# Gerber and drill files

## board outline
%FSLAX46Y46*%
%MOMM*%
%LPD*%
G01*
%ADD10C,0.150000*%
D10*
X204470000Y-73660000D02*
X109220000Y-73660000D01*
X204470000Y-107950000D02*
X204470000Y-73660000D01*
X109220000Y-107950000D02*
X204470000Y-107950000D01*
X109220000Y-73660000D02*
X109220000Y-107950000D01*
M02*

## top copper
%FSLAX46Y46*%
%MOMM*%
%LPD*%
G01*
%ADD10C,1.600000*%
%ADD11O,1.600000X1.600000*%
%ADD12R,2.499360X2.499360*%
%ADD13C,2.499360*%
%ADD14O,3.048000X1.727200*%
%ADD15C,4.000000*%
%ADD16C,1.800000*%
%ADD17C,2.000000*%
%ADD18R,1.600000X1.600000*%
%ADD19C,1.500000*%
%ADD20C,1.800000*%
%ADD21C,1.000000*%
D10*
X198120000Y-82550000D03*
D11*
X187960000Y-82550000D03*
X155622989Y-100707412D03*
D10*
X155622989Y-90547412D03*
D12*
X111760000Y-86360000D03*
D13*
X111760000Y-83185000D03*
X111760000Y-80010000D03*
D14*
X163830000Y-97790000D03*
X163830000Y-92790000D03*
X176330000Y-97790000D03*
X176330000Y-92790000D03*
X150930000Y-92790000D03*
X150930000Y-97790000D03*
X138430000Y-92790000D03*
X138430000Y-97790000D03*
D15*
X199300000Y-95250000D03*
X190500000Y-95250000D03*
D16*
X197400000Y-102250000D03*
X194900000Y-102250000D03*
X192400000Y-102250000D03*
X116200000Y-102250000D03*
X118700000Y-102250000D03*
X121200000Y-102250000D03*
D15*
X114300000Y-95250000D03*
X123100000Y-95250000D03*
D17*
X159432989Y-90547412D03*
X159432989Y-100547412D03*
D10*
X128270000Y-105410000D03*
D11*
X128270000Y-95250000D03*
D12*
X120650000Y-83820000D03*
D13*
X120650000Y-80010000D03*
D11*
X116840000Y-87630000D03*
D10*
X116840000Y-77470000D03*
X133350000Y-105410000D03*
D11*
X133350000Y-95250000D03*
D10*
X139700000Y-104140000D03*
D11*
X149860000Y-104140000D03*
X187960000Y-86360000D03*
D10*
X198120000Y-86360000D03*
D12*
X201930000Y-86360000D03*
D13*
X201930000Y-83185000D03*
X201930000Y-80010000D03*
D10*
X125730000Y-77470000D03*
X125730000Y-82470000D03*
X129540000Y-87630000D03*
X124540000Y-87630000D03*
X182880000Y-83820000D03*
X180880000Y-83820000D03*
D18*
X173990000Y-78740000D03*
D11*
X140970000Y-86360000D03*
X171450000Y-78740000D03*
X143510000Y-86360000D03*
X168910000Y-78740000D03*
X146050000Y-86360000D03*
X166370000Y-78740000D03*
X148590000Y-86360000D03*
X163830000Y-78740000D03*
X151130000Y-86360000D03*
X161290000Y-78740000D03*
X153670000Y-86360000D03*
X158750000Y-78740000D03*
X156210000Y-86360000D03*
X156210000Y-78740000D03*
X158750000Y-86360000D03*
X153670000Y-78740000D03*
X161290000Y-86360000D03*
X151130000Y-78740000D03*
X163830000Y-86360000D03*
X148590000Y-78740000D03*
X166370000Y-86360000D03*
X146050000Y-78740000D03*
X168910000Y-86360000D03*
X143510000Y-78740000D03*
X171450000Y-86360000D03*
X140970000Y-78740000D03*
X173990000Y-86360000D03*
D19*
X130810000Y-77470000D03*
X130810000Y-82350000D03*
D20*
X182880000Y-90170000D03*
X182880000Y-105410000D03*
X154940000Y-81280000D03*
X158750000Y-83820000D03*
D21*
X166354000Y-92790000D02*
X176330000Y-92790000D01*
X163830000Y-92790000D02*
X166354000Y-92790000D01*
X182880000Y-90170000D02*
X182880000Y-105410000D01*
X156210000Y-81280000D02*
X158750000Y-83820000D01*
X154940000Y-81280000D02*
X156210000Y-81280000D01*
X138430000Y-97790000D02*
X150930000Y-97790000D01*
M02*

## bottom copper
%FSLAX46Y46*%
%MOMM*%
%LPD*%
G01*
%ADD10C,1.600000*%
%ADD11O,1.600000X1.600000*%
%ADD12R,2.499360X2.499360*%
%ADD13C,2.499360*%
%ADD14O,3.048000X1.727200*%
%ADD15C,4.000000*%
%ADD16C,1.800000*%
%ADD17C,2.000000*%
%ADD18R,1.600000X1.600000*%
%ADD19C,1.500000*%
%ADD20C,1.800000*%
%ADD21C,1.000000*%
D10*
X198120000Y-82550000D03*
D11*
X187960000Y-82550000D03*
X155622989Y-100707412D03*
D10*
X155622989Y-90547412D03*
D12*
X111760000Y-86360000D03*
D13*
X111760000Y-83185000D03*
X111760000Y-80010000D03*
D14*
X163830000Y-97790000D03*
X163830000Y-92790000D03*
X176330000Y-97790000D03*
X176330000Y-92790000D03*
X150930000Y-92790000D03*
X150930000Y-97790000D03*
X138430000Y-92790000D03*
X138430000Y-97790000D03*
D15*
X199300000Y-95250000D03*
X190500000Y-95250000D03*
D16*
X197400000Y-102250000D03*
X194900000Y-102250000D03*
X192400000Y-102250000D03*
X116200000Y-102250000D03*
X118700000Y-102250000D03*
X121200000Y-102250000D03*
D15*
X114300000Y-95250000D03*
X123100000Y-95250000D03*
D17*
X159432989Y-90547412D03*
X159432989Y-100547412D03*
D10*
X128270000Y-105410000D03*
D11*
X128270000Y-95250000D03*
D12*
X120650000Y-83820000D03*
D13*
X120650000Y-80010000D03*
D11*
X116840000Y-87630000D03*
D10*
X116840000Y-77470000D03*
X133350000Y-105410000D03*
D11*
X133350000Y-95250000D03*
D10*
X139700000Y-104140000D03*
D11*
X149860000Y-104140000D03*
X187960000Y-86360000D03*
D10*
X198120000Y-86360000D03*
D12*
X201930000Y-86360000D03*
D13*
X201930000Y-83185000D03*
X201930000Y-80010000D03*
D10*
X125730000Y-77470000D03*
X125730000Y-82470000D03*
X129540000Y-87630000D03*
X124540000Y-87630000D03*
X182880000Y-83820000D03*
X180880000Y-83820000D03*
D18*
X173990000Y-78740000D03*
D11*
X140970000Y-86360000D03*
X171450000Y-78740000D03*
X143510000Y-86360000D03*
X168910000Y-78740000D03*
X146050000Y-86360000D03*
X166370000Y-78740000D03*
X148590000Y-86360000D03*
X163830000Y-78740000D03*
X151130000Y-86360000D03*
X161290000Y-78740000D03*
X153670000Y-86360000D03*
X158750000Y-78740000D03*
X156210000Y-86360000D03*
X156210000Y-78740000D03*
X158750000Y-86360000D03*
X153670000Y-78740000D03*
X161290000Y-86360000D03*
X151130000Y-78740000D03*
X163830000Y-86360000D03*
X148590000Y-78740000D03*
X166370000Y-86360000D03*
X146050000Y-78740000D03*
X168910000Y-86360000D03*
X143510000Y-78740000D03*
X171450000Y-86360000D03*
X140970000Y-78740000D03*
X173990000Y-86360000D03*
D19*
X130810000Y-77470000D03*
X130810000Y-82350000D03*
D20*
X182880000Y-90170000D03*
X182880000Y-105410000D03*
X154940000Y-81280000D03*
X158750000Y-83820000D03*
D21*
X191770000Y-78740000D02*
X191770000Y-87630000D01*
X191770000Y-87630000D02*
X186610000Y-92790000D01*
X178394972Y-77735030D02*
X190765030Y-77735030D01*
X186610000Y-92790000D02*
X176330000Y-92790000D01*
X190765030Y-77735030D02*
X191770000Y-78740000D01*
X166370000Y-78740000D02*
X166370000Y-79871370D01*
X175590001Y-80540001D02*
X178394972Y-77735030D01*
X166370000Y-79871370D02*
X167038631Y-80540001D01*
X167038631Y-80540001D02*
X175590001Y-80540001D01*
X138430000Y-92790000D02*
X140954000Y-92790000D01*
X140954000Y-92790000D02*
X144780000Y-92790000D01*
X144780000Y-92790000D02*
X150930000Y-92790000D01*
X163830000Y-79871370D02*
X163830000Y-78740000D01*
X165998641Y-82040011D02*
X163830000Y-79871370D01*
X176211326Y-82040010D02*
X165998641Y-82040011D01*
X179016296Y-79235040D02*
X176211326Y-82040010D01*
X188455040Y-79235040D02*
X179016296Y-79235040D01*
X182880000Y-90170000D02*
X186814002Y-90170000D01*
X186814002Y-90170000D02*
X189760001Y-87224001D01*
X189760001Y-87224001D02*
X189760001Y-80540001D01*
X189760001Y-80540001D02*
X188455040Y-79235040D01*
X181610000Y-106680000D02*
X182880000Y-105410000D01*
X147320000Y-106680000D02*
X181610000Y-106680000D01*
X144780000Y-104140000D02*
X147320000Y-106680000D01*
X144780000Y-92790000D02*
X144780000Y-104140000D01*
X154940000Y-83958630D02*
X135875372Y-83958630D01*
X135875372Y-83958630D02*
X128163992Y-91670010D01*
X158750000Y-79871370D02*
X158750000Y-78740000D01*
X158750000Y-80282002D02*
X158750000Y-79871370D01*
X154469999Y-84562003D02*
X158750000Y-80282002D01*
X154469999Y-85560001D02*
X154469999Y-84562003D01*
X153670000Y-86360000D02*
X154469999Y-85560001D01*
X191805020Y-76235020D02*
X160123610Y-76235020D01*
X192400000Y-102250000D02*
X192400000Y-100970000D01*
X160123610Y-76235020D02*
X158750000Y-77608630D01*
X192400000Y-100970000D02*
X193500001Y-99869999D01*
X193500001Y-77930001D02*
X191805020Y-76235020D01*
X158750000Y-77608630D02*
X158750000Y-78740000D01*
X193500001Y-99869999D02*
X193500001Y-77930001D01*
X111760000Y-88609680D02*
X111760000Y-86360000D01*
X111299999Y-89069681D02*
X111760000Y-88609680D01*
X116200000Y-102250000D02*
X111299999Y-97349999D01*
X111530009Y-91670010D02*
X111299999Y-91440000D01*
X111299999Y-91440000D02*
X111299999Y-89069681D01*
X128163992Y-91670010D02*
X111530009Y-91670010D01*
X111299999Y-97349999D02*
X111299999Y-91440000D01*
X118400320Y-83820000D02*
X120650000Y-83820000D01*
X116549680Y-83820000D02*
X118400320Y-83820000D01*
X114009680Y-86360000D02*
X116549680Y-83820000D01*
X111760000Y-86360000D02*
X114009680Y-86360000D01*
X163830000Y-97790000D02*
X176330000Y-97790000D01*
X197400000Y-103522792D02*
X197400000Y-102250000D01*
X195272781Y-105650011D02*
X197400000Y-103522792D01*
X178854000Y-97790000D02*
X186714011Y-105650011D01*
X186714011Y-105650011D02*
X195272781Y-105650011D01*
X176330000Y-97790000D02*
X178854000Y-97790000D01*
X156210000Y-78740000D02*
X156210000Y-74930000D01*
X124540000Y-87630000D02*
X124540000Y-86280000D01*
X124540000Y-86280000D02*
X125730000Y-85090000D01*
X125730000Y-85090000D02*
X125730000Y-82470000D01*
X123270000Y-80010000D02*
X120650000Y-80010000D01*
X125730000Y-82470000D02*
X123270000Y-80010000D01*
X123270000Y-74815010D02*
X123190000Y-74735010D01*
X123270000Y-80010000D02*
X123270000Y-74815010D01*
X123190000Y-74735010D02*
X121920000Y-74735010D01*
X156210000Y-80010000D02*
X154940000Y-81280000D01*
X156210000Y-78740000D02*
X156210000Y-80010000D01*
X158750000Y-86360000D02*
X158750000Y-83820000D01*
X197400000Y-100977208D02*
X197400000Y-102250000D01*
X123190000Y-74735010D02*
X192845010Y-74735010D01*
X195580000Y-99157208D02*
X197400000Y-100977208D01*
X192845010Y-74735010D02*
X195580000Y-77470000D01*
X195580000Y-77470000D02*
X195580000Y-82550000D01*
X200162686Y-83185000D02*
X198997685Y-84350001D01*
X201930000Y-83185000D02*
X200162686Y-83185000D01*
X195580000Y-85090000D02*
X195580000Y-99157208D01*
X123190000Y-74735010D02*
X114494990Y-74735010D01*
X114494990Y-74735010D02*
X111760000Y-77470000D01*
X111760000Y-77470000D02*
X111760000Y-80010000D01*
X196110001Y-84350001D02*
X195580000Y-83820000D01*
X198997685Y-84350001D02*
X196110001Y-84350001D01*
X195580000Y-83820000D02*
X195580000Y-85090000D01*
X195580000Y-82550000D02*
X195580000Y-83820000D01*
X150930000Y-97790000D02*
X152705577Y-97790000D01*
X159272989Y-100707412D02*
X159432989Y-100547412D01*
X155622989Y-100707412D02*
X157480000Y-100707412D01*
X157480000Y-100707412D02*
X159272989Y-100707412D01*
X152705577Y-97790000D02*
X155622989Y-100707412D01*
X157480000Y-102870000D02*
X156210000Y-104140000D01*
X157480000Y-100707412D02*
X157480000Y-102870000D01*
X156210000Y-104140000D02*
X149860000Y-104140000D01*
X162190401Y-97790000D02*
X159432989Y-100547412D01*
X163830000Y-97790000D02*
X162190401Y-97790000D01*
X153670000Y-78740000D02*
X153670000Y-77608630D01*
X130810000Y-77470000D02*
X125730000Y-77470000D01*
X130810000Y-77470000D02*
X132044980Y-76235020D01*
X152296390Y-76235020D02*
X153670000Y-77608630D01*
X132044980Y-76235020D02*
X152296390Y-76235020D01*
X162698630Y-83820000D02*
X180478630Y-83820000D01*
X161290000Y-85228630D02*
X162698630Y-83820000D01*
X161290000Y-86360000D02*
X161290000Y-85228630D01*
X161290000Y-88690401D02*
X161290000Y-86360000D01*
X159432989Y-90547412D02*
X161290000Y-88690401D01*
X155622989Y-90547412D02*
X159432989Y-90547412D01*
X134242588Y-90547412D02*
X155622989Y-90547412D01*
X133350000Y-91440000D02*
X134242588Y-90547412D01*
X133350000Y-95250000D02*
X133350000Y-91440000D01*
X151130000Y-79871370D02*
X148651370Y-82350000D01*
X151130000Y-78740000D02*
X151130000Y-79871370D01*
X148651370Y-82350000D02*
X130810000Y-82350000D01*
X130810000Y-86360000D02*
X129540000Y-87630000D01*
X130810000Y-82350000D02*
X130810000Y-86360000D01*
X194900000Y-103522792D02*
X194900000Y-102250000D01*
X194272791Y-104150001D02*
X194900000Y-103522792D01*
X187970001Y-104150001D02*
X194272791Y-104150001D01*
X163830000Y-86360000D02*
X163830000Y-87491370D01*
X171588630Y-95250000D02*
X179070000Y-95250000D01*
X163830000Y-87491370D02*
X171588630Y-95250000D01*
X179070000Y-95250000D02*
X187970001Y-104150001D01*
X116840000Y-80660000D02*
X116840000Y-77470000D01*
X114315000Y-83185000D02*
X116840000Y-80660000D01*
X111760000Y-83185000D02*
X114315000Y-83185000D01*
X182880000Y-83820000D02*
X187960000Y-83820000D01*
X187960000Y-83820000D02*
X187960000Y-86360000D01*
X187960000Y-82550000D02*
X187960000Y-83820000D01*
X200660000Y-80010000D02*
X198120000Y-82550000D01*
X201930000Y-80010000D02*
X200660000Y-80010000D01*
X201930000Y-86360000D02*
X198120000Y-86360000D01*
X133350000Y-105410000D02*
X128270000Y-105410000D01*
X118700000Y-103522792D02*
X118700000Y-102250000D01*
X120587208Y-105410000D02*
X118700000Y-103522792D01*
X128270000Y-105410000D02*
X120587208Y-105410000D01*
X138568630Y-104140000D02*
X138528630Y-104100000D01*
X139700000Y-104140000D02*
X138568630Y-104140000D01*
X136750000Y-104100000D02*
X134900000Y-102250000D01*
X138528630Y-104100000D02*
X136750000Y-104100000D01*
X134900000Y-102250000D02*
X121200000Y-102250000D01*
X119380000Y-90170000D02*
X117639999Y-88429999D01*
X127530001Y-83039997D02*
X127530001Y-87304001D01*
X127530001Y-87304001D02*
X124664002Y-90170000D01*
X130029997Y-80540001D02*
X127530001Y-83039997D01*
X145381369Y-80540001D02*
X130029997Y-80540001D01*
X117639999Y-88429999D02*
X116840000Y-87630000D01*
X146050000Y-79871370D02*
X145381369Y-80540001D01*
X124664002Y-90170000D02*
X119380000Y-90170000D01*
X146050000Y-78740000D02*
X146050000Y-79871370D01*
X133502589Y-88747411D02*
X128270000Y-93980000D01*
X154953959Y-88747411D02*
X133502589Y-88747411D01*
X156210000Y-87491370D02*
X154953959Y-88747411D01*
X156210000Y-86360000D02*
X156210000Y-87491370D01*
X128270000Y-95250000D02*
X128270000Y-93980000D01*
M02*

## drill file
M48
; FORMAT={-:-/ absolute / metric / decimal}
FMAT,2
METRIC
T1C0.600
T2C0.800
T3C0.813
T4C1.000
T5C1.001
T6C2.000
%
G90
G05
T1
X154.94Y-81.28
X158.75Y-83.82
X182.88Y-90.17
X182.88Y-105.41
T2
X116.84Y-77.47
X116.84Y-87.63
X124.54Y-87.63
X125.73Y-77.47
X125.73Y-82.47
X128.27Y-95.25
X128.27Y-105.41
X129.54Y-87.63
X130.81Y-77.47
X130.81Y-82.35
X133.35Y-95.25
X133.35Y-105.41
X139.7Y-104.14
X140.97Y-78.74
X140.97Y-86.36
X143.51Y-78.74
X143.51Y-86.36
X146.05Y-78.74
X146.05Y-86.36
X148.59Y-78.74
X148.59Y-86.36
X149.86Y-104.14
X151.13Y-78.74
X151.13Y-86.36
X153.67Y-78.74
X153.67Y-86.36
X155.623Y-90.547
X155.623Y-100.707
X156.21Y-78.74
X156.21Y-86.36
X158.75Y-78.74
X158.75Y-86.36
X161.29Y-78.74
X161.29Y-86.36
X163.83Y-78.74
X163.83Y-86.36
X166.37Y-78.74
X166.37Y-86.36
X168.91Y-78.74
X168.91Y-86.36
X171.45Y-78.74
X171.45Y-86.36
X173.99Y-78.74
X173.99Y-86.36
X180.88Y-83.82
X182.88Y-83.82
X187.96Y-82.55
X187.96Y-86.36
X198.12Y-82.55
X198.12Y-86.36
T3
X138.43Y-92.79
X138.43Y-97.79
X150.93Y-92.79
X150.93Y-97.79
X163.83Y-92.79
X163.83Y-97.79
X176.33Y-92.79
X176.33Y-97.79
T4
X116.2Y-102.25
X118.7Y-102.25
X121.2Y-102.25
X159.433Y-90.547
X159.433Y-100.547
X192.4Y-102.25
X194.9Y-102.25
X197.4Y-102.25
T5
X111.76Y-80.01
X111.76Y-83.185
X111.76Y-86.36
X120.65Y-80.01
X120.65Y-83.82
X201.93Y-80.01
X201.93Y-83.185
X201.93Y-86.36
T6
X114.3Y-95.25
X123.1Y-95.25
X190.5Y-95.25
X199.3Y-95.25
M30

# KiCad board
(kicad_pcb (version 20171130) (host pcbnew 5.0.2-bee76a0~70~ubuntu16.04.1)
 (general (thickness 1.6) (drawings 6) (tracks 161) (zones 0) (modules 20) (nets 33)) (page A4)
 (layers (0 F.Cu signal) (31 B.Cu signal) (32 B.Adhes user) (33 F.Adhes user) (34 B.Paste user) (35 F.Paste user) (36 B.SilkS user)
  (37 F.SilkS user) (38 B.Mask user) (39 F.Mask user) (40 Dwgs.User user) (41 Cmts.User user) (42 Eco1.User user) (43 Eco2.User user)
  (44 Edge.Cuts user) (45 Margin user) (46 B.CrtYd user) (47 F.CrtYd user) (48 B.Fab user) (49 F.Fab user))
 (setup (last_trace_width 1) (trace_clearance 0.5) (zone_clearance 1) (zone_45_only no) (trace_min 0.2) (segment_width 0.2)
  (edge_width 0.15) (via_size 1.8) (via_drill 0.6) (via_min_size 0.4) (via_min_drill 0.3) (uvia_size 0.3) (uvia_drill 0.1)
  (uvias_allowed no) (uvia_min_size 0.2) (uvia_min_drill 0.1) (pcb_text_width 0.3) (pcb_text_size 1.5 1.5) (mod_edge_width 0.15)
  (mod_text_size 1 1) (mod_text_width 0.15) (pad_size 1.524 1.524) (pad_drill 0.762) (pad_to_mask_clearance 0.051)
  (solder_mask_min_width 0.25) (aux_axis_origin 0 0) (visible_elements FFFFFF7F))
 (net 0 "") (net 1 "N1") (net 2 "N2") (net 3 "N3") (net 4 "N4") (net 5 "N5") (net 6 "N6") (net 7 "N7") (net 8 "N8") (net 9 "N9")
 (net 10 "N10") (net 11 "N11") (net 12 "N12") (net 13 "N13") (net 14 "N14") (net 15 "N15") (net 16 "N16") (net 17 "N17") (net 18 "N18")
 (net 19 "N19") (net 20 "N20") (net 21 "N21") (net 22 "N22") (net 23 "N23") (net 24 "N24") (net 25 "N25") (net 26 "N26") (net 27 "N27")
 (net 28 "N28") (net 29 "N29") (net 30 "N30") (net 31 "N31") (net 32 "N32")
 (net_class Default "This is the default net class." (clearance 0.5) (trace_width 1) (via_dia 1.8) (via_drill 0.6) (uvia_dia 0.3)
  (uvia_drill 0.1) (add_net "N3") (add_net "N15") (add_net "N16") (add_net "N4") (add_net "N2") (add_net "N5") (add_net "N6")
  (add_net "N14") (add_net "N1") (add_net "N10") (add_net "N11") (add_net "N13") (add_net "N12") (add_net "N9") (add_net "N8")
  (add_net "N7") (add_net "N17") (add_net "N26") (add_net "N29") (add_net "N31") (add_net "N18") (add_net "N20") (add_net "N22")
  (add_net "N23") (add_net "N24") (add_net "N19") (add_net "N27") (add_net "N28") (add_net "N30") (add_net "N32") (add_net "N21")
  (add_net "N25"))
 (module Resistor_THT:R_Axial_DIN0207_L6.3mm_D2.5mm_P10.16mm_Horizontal (layer F.Cu) (at 198.12 82.55 180)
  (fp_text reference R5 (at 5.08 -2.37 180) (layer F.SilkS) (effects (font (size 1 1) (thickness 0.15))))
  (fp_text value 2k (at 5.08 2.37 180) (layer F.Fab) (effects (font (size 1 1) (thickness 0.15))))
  (pad 1 thru_hole circle (at 0 0 180) (size 1.6 1.6) (drill 0.8) (layers *.Cu *.Mask) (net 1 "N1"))
  (pad 2 thru_hole oval (at 10.16 0 180) (size 1.6 1.6) (drill 0.8) (layers *.Cu *.Mask) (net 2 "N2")))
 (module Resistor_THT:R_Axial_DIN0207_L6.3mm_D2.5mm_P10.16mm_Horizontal (layer F.Cu) (at 155.622989 90.547412 270)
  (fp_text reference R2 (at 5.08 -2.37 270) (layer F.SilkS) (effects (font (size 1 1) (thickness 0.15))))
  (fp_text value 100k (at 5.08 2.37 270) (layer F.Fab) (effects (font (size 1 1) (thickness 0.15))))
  (pad 2 thru_hole oval (at 10.16 0 270) (size 1.6 1.6) (drill 0.8) (layers *.Cu *.Mask) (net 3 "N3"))
  (pad 1 thru_hole circle (at 0 0 270) (size 1.6 1.6) (drill 0.8) (layers *.Cu *.Mask) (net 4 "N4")))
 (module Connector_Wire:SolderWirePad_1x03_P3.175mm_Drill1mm (layer F.Cu) (at 111.76 86.36 90)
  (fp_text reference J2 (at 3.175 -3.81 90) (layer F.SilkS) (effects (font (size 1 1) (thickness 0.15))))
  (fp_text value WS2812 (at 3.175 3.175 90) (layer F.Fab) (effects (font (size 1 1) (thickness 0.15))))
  (pad 1 thru_hole rect (at 0 0 90) (size 2.49936 2.49936) (drill 1.00076) (layers *.Cu *.Mask) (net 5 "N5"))
  (pad 2 thru_hole circle (at 3.175 0 90) (size 2.49936 2.49936) (drill 1.00076) (layers *.Cu *.Mask) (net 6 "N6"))
  (pad 3 thru_hole circle (at 6.35 0 90) (size 2.49936 2.49936) (drill 1.00076) (layers *.Cu *.Mask) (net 3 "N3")))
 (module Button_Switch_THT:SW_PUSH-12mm (layer F.Cu) (at 163.83 92.79)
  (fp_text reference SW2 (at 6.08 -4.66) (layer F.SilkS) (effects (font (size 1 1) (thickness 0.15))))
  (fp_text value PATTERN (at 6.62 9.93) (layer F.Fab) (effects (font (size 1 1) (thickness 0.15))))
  (pad 2 thru_hole oval (at 0 5) (size 3.048 1.7272) (drill 0.8128) (layers *.Cu *.Mask) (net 3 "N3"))
  (pad 1 thru_hole oval (at 0 0) (size 3.048 1.7272) (drill 0.8128) (layers *.Cu *.Mask) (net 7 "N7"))
  (pad 2 thru_hole oval (at 12.5 5) (size 3.048 1.7272) (drill 0.8128) (layers *.Cu *.Mask) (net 3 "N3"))
  (pad 1 thru_hole oval (at 12.5 0) (size 3.048 1.7272) (drill 0.8128) (layers *.Cu *.Mask) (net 7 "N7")))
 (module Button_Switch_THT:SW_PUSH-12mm (layer F.Cu) (at 138.43 92.79)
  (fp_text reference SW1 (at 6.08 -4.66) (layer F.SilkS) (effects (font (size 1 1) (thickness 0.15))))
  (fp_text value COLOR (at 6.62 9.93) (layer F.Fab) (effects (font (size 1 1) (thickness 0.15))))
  (pad 1 thru_hole oval (at 12.5 0) (size 3.048 1.7272) (drill 0.8128) (layers *.Cu *.Mask) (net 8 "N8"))
  (pad 2 thru_hole oval (at 12.5 5) (size 3.048 1.7272) (drill 0.8128) (layers *.Cu *.Mask) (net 3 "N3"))
  (pad 1 thru_hole oval (at 0 0) (size 3.048 1.7272) (drill 0.8128) (layers *.Cu *.Mask) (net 8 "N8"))
  (pad 2 thru_hole oval (at 0 5) (size 3.048 1.7272) (drill 0.8128) (layers *.Cu *.Mask) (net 3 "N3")))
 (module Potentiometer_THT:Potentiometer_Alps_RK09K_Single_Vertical (layer F.Cu) (at 197.4 102.25 90)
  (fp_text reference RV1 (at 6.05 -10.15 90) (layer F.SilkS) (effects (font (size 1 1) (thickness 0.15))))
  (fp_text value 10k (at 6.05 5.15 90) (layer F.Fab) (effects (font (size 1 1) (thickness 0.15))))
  (pad "" np_thru_hole circle (at 7 1.9 90) (size 4 4) (drill 2) (layers *.Cu *.Mask))
  (pad "" np_thru_hole circle (at 7 -6.9 90) (size 4 4) (drill 2) (layers *.Cu *.Mask))
  (pad 1 thru_hole circle (at 0 0 90) (size 1.8 1.8) (drill 1) (layers *.Cu *.Mask) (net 3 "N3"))
  (pad 2 thru_hole circle (at 0 -2.5 90) (size 1.8 1.8) (drill 1) (layers *.Cu *.Mask) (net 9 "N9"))
  (pad 3 thru_hole circle (at 0 -5 90) (size 1.8 1.8) (drill 1) (layers *.Cu *.Mask) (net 5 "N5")))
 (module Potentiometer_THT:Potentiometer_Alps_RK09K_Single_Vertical (layer F.Cu) (at 121.2 102.25 90)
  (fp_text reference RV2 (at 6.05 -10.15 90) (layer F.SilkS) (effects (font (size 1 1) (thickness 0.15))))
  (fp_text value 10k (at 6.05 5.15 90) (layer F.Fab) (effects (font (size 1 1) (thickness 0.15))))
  (pad 3 thru_hole circle (at 0 -5 90) (size 1.8 1.8) (drill 1) (layers *.Cu *.Mask) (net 5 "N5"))
  (pad 2 thru_hole circle (at 0 -2.5 90) (size 1.8 1.8) (drill 1) (layers *.Cu *.Mask) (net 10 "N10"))
  (pad 1 thru_hole circle (at 0 0 90) (size 1.8 1.8) (drill 1) (layers *.Cu *.Mask) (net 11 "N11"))
  (pad "" np_thru_hole circle (at 7 -6.9 90) (size 4 4) (drill 2) (layers *.Cu *.Mask))
  (pad "" np_thru_hole circle (at 7 1.9 90) (size 4 4) (drill 2) (layers *.Cu *.Mask)))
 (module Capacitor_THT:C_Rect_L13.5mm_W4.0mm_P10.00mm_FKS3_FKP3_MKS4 (layer F.Cu) (at 159.432989 90.547412 270)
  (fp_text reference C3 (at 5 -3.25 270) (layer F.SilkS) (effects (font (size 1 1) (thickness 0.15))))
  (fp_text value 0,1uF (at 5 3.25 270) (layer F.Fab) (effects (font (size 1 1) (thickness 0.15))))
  (pad 1 thru_hole circle (at 0 0 270) (size 2 2) (drill 1) (layers *.Cu *.Mask) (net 4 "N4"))
  (pad 2 thru_hole circle (at 10 0 270) (size 2 2) (drill 1) (layers *.Cu *.Mask) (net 3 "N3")))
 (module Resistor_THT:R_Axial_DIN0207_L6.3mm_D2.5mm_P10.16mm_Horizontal (layer F.Cu) (at 128.27 105.41 90)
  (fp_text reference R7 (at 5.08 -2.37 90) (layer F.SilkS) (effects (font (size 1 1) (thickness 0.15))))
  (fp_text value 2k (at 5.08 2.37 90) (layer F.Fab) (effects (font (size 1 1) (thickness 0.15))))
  (pad 1 thru_hole circle (at 0 0 90) (size 1.6 1.6) (drill 0.8) (layers *.Cu *.Mask) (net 10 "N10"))
  (pad 2 thru_hole oval (at 10.16 0 90) (size 1.6 1.6) (drill 0.8) (layers *.Cu *.Mask) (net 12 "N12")))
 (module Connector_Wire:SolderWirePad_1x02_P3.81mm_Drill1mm (layer F.Cu) (at 120.65 83.82 90)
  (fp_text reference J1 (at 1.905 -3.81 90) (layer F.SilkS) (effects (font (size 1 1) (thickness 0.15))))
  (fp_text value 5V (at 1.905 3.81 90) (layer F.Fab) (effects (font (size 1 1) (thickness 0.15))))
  (pad 1 thru_hole rect (at 0 0 90) (size 2.49936 2.49936) (drill 1.00076) (layers *.Cu *.Mask) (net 5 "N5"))
  (pad 2 thru_hole circle (at 3.81 0 90) (size 2.49936 2.49936) (drill 1.00076) (layers *.Cu *.Mask) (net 3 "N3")))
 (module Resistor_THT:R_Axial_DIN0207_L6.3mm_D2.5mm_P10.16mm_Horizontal (layer F.Cu) (at 116.84 77.47 270)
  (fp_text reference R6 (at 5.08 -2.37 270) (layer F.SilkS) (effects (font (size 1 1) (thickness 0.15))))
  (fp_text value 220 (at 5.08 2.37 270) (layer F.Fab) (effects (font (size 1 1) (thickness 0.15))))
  (pad 2 thru_hole oval (at 10.16 0 270) (size 1.6 1.6) (drill 0.8) (layers *.Cu *.Mask) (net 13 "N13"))
  (pad 1 thru_hole circle (at 0 0 270) (size 1.6 1.6) (drill 0.8) (layers *.Cu *.Mask) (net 6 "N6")))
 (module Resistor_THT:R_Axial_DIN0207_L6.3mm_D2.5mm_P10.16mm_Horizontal (layer F.Cu) (at 133.35 105.41 90)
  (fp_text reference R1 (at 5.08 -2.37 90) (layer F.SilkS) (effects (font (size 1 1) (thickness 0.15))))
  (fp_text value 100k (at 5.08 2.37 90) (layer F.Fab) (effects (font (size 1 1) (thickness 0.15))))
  (pad 1 thru_hole circle (at 0 0 90) (size 1.6 1.6) (drill 0.8) (layers *.Cu *.Mask) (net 10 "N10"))
  (pad 2 thru_hole oval (at 10.16 0 90) (size 1.6 1.6) (drill 0.8) (layers *.Cu *.Mask) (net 4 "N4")))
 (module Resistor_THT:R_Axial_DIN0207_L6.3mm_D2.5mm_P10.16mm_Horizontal (layer F.Cu) (at 139.7 104.14)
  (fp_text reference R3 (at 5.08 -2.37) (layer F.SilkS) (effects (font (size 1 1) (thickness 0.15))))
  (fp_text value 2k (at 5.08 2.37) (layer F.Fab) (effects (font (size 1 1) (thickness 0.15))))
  (pad 1 thru_hole circle (at 0 0) (size 1.6 1.6) (drill 0.8) (layers *.Cu *.Mask) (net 11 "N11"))
  (pad 2 thru_hole oval (at 10.16 0) (size 1.6 1.6) (drill 0.8) (layers *.Cu *.Mask) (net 3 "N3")))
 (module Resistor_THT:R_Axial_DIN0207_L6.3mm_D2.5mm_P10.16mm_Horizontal (layer F.Cu) (at 198.12 86.36 180)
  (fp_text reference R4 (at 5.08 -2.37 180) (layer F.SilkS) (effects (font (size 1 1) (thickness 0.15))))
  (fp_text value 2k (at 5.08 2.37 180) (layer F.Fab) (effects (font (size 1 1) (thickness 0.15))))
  (pad 2 thru_hole oval (at 10.16 0 180) (size 1.6 1.6) (drill 0.8) (layers *.Cu *.Mask) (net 2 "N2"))
  (pad 1 thru_hole circle (at 0 0 180) (size 1.6 1.6) (drill 0.8) (layers *.Cu *.Mask) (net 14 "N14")))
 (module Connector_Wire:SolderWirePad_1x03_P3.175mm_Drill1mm (layer F.Cu) (at 201.93 86.36 90)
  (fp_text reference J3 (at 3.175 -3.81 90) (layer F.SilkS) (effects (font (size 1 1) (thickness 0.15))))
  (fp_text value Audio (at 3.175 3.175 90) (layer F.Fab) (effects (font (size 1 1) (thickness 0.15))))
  (pad 1 thru_hole rect (at 0 0 90) (size 2.49936 2.49936) (drill 1.00076) (layers *.Cu *.Mask) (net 14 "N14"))
  (pad 2 thru_hole circle (at 3.175 0 90) (size 2.49936 2.49936) (drill 1.00076) (layers *.Cu *.Mask) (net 3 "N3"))
  (pad 3 thru_hole circle (at 6.35 0 90) (size 2.49936 2.49936) (drill 1.00076) (layers *.Cu *.Mask) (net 1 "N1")))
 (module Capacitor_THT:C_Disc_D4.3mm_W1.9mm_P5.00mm (layer F.Cu) (at 125.73 82.47 90)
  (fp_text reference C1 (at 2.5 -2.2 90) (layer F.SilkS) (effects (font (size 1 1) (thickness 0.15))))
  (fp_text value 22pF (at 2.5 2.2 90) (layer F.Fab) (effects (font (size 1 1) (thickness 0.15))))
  (pad 2 thru_hole circle (at 5 0 90) (size 1.6 1.6) (drill 0.8) (layers *.Cu *.Mask) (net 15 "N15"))
  (pad 1 thru_hole circle (at 0 0 90) (size 1.6 1.6) (drill 0.8) (layers *.Cu *.Mask) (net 3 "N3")))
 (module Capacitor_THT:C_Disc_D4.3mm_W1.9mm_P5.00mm (layer F.Cu) (at 129.54 87.63 180)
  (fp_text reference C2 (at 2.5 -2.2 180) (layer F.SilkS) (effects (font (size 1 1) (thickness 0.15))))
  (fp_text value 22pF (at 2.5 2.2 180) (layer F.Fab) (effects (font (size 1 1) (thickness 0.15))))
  (pad 1 thru_hole circle (at 0 0 180) (size 1.6 1.6) (drill 0.8) (layers *.Cu *.Mask) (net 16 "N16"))
  (pad 2 thru_hole circle (at 5 0 180) (size 1.6 1.6) (drill 0.8) (layers *.Cu *.Mask) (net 3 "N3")))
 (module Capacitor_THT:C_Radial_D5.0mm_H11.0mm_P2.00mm (layer F.Cu) (at 182.88 83.82 180)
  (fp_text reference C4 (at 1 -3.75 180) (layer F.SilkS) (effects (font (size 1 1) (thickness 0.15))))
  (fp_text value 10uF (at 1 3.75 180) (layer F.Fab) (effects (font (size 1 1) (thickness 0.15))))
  (pad 1 thru_hole circle (at 0 0 180) (size 1.6 1.6) (drill 0.8) (layers *.Cu *.Mask) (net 2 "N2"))
  (pad 2 thru_hole circle (at 2 0 180) (size 1.6 1.6) (drill 0.8) (layers *.Cu *.Mask) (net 4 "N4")))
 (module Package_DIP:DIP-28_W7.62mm (layer F.Cu) (at 173.99 78.74 270)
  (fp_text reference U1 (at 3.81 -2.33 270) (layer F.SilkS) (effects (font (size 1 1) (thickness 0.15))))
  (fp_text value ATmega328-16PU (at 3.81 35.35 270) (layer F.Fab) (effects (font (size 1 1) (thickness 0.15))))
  (pad 1 thru_hole rect (at 0 0 270) (size 1.6 1.6) (drill 0.8) (layers *.Cu *.Mask) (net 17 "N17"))
  (pad 15 thru_hole oval (at 7.62 33.02 270) (size 1.6 1.6) (drill 0.8) (layers *.Cu *.Mask) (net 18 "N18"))
  (pad 2 thru_hole oval (at 0 2.54 270) (size 1.6 1.6) (drill 0.8) (layers *.Cu *.Mask) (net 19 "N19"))
  (pad 16 thru_hole oval (at 7.62 30.48 270) (size 1.6 1.6) (drill 0.8) (layers *.Cu *.Mask) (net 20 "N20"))
  (pad 3 thru_hole oval (at 0 5.08 270) (size 1.6 1.6) (drill 0.8) (layers *.Cu *.Mask) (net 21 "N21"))
  (pad 17 thru_hole oval (at 7.62 27.94 270) (size 1.6 1.6) (drill 0.8) (layers *.Cu *.Mask) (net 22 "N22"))
  (pad 4 thru_hole oval (at 0 7.62 270) (size 1.6 1.6) (drill 0.8) (layers *.Cu *.Mask) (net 7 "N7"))
  (pad 18 thru_hole oval (at 7.62 25.4 270) (size 1.6 1.6) (drill 0.8) (layers *.Cu *.Mask) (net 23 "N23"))
  (pad 5 thru_hole oval (at 0 10.16 270) (size 1.6 1.6) (drill 0.8) (layers *.Cu *.Mask) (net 8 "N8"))
  (pad 19 thru_hole oval (at 7.62 22.86 270) (size 1.6 1.6) (drill 0.8) (layers *.Cu *.Mask) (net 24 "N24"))
  (pad 6 thru_hole oval (at 0 12.7 270) (size 1.6 1.6) (drill 0.8) (layers *.Cu *.Mask) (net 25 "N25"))
  (pad 20 thru_hole oval (at 7.62 20.32 270) (size 1.6 1.6) (drill 0.8) (layers *.Cu *.Mask) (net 5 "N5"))
  (pad 7 thru_hole oval (at 0 15.24 270) (size 1.6 1.6) (drill 0.8) (layers *.Cu *.Mask) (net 5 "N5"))
  (pad 21 thru_hole oval (at 7.62 17.78 270) (size 1.6 1.6) (drill 0.8) (layers *.Cu *.Mask) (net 12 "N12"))
  (pad 8 thru_hole oval (at 0 17.78 270) (size 1.6 1.6) (drill 0.8) (layers *.Cu *.Mask) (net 3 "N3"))
  (pad 22 thru_hole oval (at 7.62 15.24 270) (size 1.6 1.6) (drill 0.8) (layers *.Cu *.Mask) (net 3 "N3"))
  (pad 9 thru_hole oval (at 0 20.32 270) (size 1.6 1.6) (drill 0.8) (layers *.Cu *.Mask) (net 15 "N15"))
  (pad 23 thru_hole oval (at 7.62 12.7 270) (size 1.6 1.6) (drill 0.8) (layers *.Cu *.Mask) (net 4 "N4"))
  (pad 10 thru_hole oval (at 0 22.86 270) (size 1.6 1.6) (drill 0.8) (layers *.Cu *.Mask) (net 16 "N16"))
  (pad 24 thru_hole oval (at 7.62 10.16 270) (size 1.6 1.6) (drill 0.8) (layers *.Cu *.Mask) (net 9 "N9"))
  (pad 11 thru_hole oval (at 0 25.4 270) (size 1.6 1.6) (drill 0.8) (layers *.Cu *.Mask) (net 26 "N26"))
  (pad 25 thru_hole oval (at 7.62 7.62 270) (size 1.6 1.6) (drill 0.8) (layers *.Cu *.Mask) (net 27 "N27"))
  (pad 12 thru_hole oval (at 0 27.94 270) (size 1.6 1.6) (drill 0.8) (layers *.Cu *.Mask) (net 13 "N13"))
  (pad 26 thru_hole oval (at 7.62 5.08 270) (size 1.6 1.6) (drill 0.8) (layers *.Cu *.Mask) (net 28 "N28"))
  (pad 13 thru_hole oval (at 0 30.48 270) (size 1.6 1.6) (drill 0.8) (layers *.Cu *.Mask) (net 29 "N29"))
  (pad 27 thru_hole oval (at 7.62 2.54 270) (size 1.6 1.6) (drill 0.8) (layers *.Cu *.Mask) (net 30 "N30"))
  (pad 14 thru_hole oval (at 0 33.02 270) (size 1.6 1.6) (drill 0.8) (layers *.Cu *.Mask) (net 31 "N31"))
  (pad 28 thru_hole oval (at 7.62 0 270) (size 1.6 1.6) (drill 0.8) (layers *.Cu *.Mask) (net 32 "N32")))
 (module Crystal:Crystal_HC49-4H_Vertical (layer F.Cu) (at 130.81 77.47 270)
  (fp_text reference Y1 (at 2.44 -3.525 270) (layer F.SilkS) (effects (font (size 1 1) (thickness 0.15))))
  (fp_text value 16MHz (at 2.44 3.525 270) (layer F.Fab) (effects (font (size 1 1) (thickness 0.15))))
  (pad 1 thru_hole circle (at 0 0 270) (size 1.5 1.5) (drill 0.8) (layers *.Cu *.Mask) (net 15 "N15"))
  (pad 2 thru_hole circle (at 4.88 0 270) (size 1.5 1.5) (drill 0.8) (layers *.Cu *.Mask) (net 16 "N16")))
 (gr_line (start 204.47 73.66) (end 109.22 73.66) (layer Edge.Cuts) (width 0.15))
 (gr_line (start 204.47 107.95) (end 204.47 73.66) (layer Edge.Cuts) (width 0.15))
 (gr_line (start 109.22 107.95) (end 204.47 107.95) (layer Edge.Cuts) (width 0.15))
 (gr_line (start 109.22 73.66) (end 109.22 107.95) (layer Edge.Cuts) (width 0.15))
 (segment (start 166.354 92.79) (end 176.33 92.79) (width 1) (layer F.Cu) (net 7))
 (segment (start 163.83 92.79) (end 166.354 92.79) (width 1) (layer F.Cu) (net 7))
 (segment (start 191.77 78.74) (end 191.77 87.63) (width 1) (layer B.Cu) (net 7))
 (segment (start 191.77 87.63) (end 186.61 92.79) (width 1) (layer B.Cu) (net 7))
 (segment (start 178.394972 77.73503) (end 190.76503 77.73503) (width 1) (layer B.Cu) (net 7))
 (segment (start 186.61 92.79) (end 176.33 92.79) (width 1) (layer B.Cu) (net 7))
 (segment (start 190.76503 77.73503) (end 191.77 78.74) (width 1) (layer B.Cu) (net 7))
 (segment (start 166.37 78.74) (end 166.37 79.87137) (width 1) (layer B.Cu) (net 7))
 (segment (start 175.590001 80.540001) (end 178.394972 77.73503) (width 1) (layer B.Cu) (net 7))
 (segment (start 166.37 79.87137) (end 167.038631 80.540001) (width 1) (layer B.Cu) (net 7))
 (segment (start 167.038631 80.540001) (end 175.590001 80.540001) (width 1) (layer B.Cu) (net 7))
 (via (at 182.88 90.17) (size 1.8) (drill 0.6) (layers F.Cu B.Cu) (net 8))
 (via (at 182.88 105.41) (size 1.8) (drill 0.6) (layers F.Cu B.Cu) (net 8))
 (segment (start 138.43 92.79) (end 140.954 92.79) (width 1) (layer B.Cu) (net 8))
 (segment (start 140.954 92.79) (end 144.78 92.79) (width 1) (layer B.Cu) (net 8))
 (segment (start 144.78 92.79) (end 150.93 92.79) (width 1) (layer B.Cu) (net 8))
 (segment (start 163.83 79.87137) (end 163.83 78.74) (width 1) (layer B.Cu) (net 8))
 (segment (start 165.998641 82.040011) (end 163.83 79.87137) (width 1) (layer B.Cu) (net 8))
 (segment (start 176.211326 82.04001) (end 165.998641 82.040011) (width 1) (layer B.Cu) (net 8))
 (segment (start 179.016296 79.23504) (end 176.211326 82.04001) (width 1) (layer B.Cu) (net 8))
 (segment (start 188.45504 79.23504) (end 179.016296 79.23504) (width 1) (layer B.Cu) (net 8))
 (segment (start 182.88 90.17) (end 186.814002 90.17) (width 1) (layer B.Cu) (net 8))
 (segment (start 186.814002 90.17) (end 189.760001 87.224001) (width 1) (layer B.Cu) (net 8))
 (segment (start 189.760001 87.224001) (end 189.760001 80.540001) (width 1) (layer B.Cu) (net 8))
 (segment (start 189.760001 80.540001) (end 188.45504 79.23504) (width 1) (layer B.Cu) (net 8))
 (segment (start 182.88 90.17) (end 182.88 105.41) (width 1) (layer F.Cu) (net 8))
 (segment (start 181.61 106.68) (end 182.88 105.41) (width 1) (layer B.Cu) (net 8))
 (segment (start 147.32 106.68) (end 181.61 106.68) (width 1) (layer B.Cu) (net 8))
 (segment (start 144.78 104.14) (end 147.32 106.68) (width 1) (layer B.Cu) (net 8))
 (segment (start 144.78 92.79) (end 144.78 104.14) (width 1) (layer B.Cu) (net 8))
 (segment (start 154.94 83.95863) (end 135.875372 83.95863) (width 1) (layer B.Cu) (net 5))
 (segment (start 135.875372 83.95863) (end 128.163992 91.67001) (width 1) (layer B.Cu) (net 5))
 (segment (start 158.75 79.87137) (end 158.75 78.74) (width 1) (layer B.Cu) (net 5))
 (segment (start 158.75 80.282002) (end 158.75 79.87137) (width 1) (layer B.Cu) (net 5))
 (segment (start 154.469999 84.562003) (end 158.75 80.282002) (width 1) (layer B.Cu) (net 5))
 (segment (start 154.469999 85.560001) (end 154.469999 84.562003) (width 1) (layer B.Cu) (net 5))
 (segment (start 153.67 86.36) (end 154.469999 85.560001) (width 1) (layer B.Cu) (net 5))
 (segment (start 191.80502 76.23502) (end 160.12361 76.23502) (width 1) (layer B.Cu) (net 5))
 (segment (start 192.4 102.25) (end 192.4 100.97) (width 1) (layer B.Cu) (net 5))
 (segment (start 160.12361 76.23502) (end 158.75 77.60863) (width 1) (layer B.Cu) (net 5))
 (segment (start 192.4 100.97) (end 193.500001 99.869999) (width 1) (layer B.Cu) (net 5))
 (segment (start 193.500001 77.930001) (end 191.80502 76.23502) (width 1) (layer B.Cu) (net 5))
 (segment (start 158.75 77.60863) (end 158.75 78.74) (width 1) (layer B.Cu) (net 5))
 (segment (start 193.500001 99.869999) (end 193.500001 77.930001) (width 1) (layer B.Cu) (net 5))
 (segment (start 111.76 88.60968) (end 111.76 86.36) (width 1) (layer B.Cu) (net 5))
 (segment (start 111.299999 89.069681) (end 111.76 88.60968) (width 1) (layer B.Cu) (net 5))
 (segment (start 116.2 102.25) (end 111.299999 97.349999) (width 1) (layer B.Cu) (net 5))
 (segment (start 111.530009 91.67001) (end 111.299999 91.44) (width 1) (layer B.Cu) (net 5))
 (segment (start 111.299999 91.44) (end 111.299999 89.069681) (width 1) (layer B.Cu) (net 5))
 (segment (start 128.163992 91.67001) (end 111.530009 91.67001) (width 1) (layer B.Cu) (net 5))
 (segment (start 111.299999 97.349999) (end 111.299999 91.44) (width 1) (layer B.Cu) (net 5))
 (segment (start 118.40032 83.82) (end 120.65 83.82) (width 1) (layer B.Cu) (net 5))
 (segment (start 116.54968 83.82) (end 118.40032 83.82) (width 1) (layer B.Cu) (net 5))
 (segment (start 114.00968 86.36) (end 116.54968 83.82) (width 1) (layer B.Cu) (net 5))
 (segment (start 111.76 86.36) (end 114.00968 86.36) (width 1) (layer B.Cu) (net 5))
 (via (at 154.94 81.28) (size 1.8) (drill 0.6) (layers F.Cu B.Cu) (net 3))
 (via (at 158.75 83.82) (size 1.8) (drill 0.6) (layers F.Cu B.Cu) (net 3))
 (segment (start 163.83 97.79) (end 176.33 97.79) (width 1) (layer B.Cu) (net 3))
 (segment (start 197.4 103.522792) (end 197.4 102.25) (width 1) (layer B.Cu) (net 3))
 (segment (start 195.272781 105.650011) (end 197.4 103.522792) (width 1) (layer B.Cu) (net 3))
 (segment (start 178.854 97.79) (end 186.714011 105.650011) (width 1) (layer B.Cu) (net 3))
 (segment (start 186.714011 105.650011) (end 195.272781 105.650011) (width 1) (layer B.Cu) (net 3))
 (segment (start 176.33 97.79) (end 178.854 97.79) (width 1) (layer B.Cu) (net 3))
 (segment (start 156.21 78.74) (end 156.21 74.93) (width 1) (layer B.Cu) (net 3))
 (segment (start 124.54 87.63) (end 124.54 86.28) (width 1) (layer B.Cu) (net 3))
 (segment (start 124.54 86.28) (end 125.73 85.09) (width 1) (layer B.Cu) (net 3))
 (segment (start 125.73 85.09) (end 125.73 82.47) (width 1) (layer B.Cu) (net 3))
 (segment (start 123.27 80.01) (end 120.65 80.01) (width 1) (layer B.Cu) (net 3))
 (segment (start 125.73 82.47) (end 123.27 80.01) (width 1) (layer B.Cu) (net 3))
 (segment (start 123.27 74.81501) (end 123.19 74.73501) (width 1) (layer B.Cu) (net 3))
 (segment (start 123.27 80.01) (end 123.27 74.81501) (width 1) (layer B.Cu) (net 3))
 (segment (start 123.19 74.73501) (end 121.92 74.73501) (width 1) (layer B.Cu) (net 3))
 (segment (start 156.21 81.28) (end 158.75 83.82) (width 1) (layer F.Cu) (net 3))
 (segment (start 154.94 81.28) (end 156.21 81.28) (width 1) (layer F.Cu) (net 3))
 (segment (start 156.21 80.01) (end 154.94 81.28) (width 1) (layer B.Cu) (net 3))
 (segment (start 156.21 78.74) (end 156.21 80.01) (width 1) (layer B.Cu) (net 3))
 (segment (start 158.75 86.36) (end 158.75 83.82) (width 1) (layer B.Cu) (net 3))
 (segment (start 197.4 100.977208) (end 197.4 102.25) (width 1) (layer B.Cu) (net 3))
 (segment (start 123.19 74.73501) (end 192.84501 74.73501) (width 1) (layer B.Cu) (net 3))
 (segment (start 195.58 99.157208) (end 197.4 100.977208) (width 1) (layer B.Cu) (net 3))
 (segment (start 192.84501 74.73501) (end 195.58 77.47) (width 1) (layer B.Cu) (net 3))
 (segment (start 195.58 77.47) (end 195.58 82.55) (width 1) (layer B.Cu) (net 3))
 (segment (start 138.43 97.79) (end 150.93 97.79) (width 1) (layer F.Cu) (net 3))
 (segment (start 200.162686 83.185) (end 198.997685 84.350001) (width 1) (layer B.Cu) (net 3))
 (segment (start 201.93 83.185) (end 200.162686 83.185) (width 1) (layer B.Cu) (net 3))
 (segment (start 195.58 85.09) (end 195.58 99.157208) (width 1) (layer B.Cu) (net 3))
 (segment (start 123.19 74.73501) (end 114.49499 74.73501) (width 1) (layer B.Cu) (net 3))
 (segment (start 114.49499 74.73501) (end 111.76 77.47) (width 1) (layer B.Cu) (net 3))
 (segment (start 111.76 77.47) (end 111.76 80.01) (width 1) (layer B.Cu) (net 3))
 (segment (start 196.110001 84.350001) (end 195.58 83.82) (width 1) (layer B.Cu) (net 3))
 (segment (start 198.997685 84.350001) (end 196.110001 84.350001) (width 1) (layer B.Cu) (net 3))
 (segment (start 195.58 83.82) (end 195.58 85.09) (width 1) (layer B.Cu) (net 3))
 (segment (start 195.58 82.55) (end 195.58 83.82) (width 1) (layer B.Cu) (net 3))
 (segment (start 150.93 97.79) (end 152.705577 97.79) (width 1) (layer B.Cu) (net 3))
 (segment (start 159.272989 100.707412) (end 159.432989 100.547412) (width 1) (layer B.Cu) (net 3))
 (segment (start 155.622989 100.707412) (end 157.48 100.707412) (width 1) (layer B.Cu) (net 3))
 (segment (start 157.48 100.707412) (end 159.272989 100.707412) (width 1) (layer B.Cu) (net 3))
 (segment (start 152.705577 97.79) (end 155.622989 100.707412) (width 1) (layer B.Cu) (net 3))
 (segment (start 157.48 102.87) (end 156.21 104.14) (width 1) (layer B.Cu) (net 3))
 (segment (start 157.48 100.707412) (end 157.48 102.87) (width 1) (layer B.Cu) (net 3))
 (segment (start 156.21 104.14) (end 149.86 104.14) (width 1) (layer B.Cu) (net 3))
 (segment (start 162.190401 97.79) (end 159.432989 100.547412) (width 1) (layer B.Cu) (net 3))
 (segment (start 163.83 97.79) (end 162.190401 97.79) (width 1) (layer B.Cu) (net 3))
 (segment (start 153.67 78.74) (end 153.67 77.60863) (width 1) (layer B.Cu) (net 15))
 (segment (start 130.81 77.47) (end 125.73 77.47) (width 1) (layer B.Cu) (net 15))
 (segment (start 130.81 77.47) (end 132.04498 76.23502) (width 1) (layer B.Cu) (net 15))
 (segment (start 152.29639 76.23502) (end 153.67 77.60863) (width 1) (layer B.Cu) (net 15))
 (segment (start 132.04498 76.23502) (end 152.29639 76.23502) (width 1) (layer B.Cu) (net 15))
 (segment (start 162.69863 83.82) (end 180.47863 83.82) (width 1) (layer B.Cu) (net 4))
 (segment (start 161.29 85.22863) (end 162.69863 83.82) (width 1) (layer B.Cu) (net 4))
 (segment (start 161.29 86.36) (end 161.29 85.22863) (width 1) (layer B.Cu) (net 4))
 (segment (start 161.29 88.690401) (end 161.29 86.36) (width 1) (layer B.Cu) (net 4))
 (segment (start 159.432989 90.547412) (end 161.29 88.690401) (width 1) (layer B.Cu) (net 4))
 (segment (start 155.622989 90.547412) (end 159.432989 90.547412) (width 1) (layer B.Cu) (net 4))
 (segment (start 134.242588 90.547412) (end 155.622989 90.547412) (width 1) (layer B.Cu) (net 4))
 (segment (start 133.35 91.44) (end 134.242588 90.547412) (width 1) (layer B.Cu) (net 4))
 (segment (start 133.35 95.25) (end 133.35 91.44) (width 1) (layer B.Cu) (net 4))
 (segment (start 151.13 79.87137) (end 148.65137 82.35) (width 1) (layer B.Cu) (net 16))
 (segment (start 151.13 78.74) (end 151.13 79.87137) (width 1) (layer B.Cu) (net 16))
 (segment (start 148.65137 82.35) (end 130.81 82.35) (width 1) (layer B.Cu) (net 16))
 (segment (start 130.81 86.36) (end 129.54 87.63) (width 1) (layer B.Cu) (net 16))
 (segment (start 130.81 82.35) (end 130.81 86.36) (width 1) (layer B.Cu) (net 16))
 (segment (start 194.9 103.522792) (end 194.9 102.25) (width 1) (layer B.Cu) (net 9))
 (segment (start 194.272791 104.150001) (end 194.9 103.522792) (width 1) (layer B.Cu) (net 9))
 (segment (start 187.970001 104.150001) (end 194.272791 104.150001) (width 1) (layer B.Cu) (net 9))
 (segment (start 163.83 86.36) (end 163.83 87.49137) (width 1) (layer B.Cu) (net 9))
 (segment (start 171.58863 95.25) (end 179.07 95.25) (width 1) (layer B.Cu) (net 9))
 (segment (start 163.83 87.49137) (end 171.58863 95.25) (width 1) (layer B.Cu) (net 9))
 (segment (start 179.07 95.25) (end 187.970001 104.150001) (width 1) (layer B.Cu) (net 9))
 (segment (start 116.84 80.66) (end 116.84 77.47) (width 1) (layer B.Cu) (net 6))
 (segment (start 114.315 83.185) (end 116.84 80.66) (width 1) (layer B.Cu) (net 6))
 (segment (start 111.76 83.185) (end 114.315 83.185) (width 1) (layer B.Cu) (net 6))
 (segment (start 182.88 83.82) (end 187.96 83.82) (width 1) (layer B.Cu) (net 2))
 (segment (start 187.96 83.82) (end 187.96 86.36) (width 1) (layer B.Cu) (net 2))
 (segment (start 187.96 82.55) (end 187.96 83.82) (width 1) (layer B.Cu) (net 2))
 (segment (start 200.66 80.01) (end 198.12 82.55) (width 1) (layer B.Cu) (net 1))
 (segment (start 201.93 80.01) (end 200.66 80.01) (width 1) (layer B.Cu) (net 1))
 (segment (start 201.93 86.36) (end 198.12 86.36) (width 1) (layer B.Cu) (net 14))
 (segment (start 133.35 105.41) (end 128.27 105.41) (width 1) (layer B.Cu) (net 10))
 (segment (start 118.7 103.522792) (end 118.7 102.25) (width 1) (layer B.Cu) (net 10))
 (segment (start 120.587208 105.41) (end 118.7 103.522792) (width 1) (layer B.Cu) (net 10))
 (segment (start 128.27 105.41) (end 120.587208 105.41) (width 1) (layer B.Cu) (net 10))
 (segment (start 138.56863 104.14) (end 138.52863 104.1) (width 1) (layer B.Cu) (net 11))
 (segment (start 139.7 104.14) (end 138.56863 104.14) (width 1) (layer B.Cu) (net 11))
 (segment (start 136.75 104.1) (end 134.9 102.25) (width 1) (layer B.Cu) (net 11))
 (segment (start 138.52863 104.1) (end 136.75 104.1) (width 1) (layer B.Cu) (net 11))
 (segment (start 134.9 102.25) (end 121.2 102.25) (width 1) (layer B.Cu) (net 11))
 (segment (start 119.38 90.17) (end 117.639999 88.429999) (width 1) (layer B.Cu) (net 13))
 (segment (start 127.530001 83.039997) (end 127.530001 87.304001) (width 1) (layer B.Cu) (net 13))
 (segment (start 127.530001 87.304001) (end 124.664002 90.17) (width 1) (layer B.Cu) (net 13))
 (segment (start 130.029997 80.540001) (end 127.530001 83.039997) (width 1) (layer B.Cu) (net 13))
 (segment (start 145.381369 80.540001) (end 130.029997 80.540001) (width 1) (layer B.Cu) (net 13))
 (segment (start 117.639999 88.429999) (end 116.84 87.63) (width 1) (layer B.Cu) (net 13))
 (segment (start 146.05 79.87137) (end 145.381369 80.540001) (width 1) (layer B.Cu) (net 13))
 (segment (start 124.664002 90.17) (end 119.38 90.17) (width 1) (layer B.Cu) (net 13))
 (segment (start 146.05 78.74) (end 146.05 79.87137) (width 1) (layer B.Cu) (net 13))
 (segment (start 133.502589 88.747411) (end 128.27 93.98) (width 1) (layer B.Cu) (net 12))
 (segment (start 154.953959 88.747411) (end 133.502589 88.747411) (width 1) (layer B.Cu) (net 12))
 (segment (start 156.21 87.49137) (end 154.953959 88.747411) (width 1) (layer B.Cu) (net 12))
 (segment (start 156.21 86.36) (end 156.21 87.49137) (width 1) (layer B.Cu) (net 12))
 (segment (start 128.27 95.25) (end 128.27 93.98) (width 1) (layer B.Cu) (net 12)))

